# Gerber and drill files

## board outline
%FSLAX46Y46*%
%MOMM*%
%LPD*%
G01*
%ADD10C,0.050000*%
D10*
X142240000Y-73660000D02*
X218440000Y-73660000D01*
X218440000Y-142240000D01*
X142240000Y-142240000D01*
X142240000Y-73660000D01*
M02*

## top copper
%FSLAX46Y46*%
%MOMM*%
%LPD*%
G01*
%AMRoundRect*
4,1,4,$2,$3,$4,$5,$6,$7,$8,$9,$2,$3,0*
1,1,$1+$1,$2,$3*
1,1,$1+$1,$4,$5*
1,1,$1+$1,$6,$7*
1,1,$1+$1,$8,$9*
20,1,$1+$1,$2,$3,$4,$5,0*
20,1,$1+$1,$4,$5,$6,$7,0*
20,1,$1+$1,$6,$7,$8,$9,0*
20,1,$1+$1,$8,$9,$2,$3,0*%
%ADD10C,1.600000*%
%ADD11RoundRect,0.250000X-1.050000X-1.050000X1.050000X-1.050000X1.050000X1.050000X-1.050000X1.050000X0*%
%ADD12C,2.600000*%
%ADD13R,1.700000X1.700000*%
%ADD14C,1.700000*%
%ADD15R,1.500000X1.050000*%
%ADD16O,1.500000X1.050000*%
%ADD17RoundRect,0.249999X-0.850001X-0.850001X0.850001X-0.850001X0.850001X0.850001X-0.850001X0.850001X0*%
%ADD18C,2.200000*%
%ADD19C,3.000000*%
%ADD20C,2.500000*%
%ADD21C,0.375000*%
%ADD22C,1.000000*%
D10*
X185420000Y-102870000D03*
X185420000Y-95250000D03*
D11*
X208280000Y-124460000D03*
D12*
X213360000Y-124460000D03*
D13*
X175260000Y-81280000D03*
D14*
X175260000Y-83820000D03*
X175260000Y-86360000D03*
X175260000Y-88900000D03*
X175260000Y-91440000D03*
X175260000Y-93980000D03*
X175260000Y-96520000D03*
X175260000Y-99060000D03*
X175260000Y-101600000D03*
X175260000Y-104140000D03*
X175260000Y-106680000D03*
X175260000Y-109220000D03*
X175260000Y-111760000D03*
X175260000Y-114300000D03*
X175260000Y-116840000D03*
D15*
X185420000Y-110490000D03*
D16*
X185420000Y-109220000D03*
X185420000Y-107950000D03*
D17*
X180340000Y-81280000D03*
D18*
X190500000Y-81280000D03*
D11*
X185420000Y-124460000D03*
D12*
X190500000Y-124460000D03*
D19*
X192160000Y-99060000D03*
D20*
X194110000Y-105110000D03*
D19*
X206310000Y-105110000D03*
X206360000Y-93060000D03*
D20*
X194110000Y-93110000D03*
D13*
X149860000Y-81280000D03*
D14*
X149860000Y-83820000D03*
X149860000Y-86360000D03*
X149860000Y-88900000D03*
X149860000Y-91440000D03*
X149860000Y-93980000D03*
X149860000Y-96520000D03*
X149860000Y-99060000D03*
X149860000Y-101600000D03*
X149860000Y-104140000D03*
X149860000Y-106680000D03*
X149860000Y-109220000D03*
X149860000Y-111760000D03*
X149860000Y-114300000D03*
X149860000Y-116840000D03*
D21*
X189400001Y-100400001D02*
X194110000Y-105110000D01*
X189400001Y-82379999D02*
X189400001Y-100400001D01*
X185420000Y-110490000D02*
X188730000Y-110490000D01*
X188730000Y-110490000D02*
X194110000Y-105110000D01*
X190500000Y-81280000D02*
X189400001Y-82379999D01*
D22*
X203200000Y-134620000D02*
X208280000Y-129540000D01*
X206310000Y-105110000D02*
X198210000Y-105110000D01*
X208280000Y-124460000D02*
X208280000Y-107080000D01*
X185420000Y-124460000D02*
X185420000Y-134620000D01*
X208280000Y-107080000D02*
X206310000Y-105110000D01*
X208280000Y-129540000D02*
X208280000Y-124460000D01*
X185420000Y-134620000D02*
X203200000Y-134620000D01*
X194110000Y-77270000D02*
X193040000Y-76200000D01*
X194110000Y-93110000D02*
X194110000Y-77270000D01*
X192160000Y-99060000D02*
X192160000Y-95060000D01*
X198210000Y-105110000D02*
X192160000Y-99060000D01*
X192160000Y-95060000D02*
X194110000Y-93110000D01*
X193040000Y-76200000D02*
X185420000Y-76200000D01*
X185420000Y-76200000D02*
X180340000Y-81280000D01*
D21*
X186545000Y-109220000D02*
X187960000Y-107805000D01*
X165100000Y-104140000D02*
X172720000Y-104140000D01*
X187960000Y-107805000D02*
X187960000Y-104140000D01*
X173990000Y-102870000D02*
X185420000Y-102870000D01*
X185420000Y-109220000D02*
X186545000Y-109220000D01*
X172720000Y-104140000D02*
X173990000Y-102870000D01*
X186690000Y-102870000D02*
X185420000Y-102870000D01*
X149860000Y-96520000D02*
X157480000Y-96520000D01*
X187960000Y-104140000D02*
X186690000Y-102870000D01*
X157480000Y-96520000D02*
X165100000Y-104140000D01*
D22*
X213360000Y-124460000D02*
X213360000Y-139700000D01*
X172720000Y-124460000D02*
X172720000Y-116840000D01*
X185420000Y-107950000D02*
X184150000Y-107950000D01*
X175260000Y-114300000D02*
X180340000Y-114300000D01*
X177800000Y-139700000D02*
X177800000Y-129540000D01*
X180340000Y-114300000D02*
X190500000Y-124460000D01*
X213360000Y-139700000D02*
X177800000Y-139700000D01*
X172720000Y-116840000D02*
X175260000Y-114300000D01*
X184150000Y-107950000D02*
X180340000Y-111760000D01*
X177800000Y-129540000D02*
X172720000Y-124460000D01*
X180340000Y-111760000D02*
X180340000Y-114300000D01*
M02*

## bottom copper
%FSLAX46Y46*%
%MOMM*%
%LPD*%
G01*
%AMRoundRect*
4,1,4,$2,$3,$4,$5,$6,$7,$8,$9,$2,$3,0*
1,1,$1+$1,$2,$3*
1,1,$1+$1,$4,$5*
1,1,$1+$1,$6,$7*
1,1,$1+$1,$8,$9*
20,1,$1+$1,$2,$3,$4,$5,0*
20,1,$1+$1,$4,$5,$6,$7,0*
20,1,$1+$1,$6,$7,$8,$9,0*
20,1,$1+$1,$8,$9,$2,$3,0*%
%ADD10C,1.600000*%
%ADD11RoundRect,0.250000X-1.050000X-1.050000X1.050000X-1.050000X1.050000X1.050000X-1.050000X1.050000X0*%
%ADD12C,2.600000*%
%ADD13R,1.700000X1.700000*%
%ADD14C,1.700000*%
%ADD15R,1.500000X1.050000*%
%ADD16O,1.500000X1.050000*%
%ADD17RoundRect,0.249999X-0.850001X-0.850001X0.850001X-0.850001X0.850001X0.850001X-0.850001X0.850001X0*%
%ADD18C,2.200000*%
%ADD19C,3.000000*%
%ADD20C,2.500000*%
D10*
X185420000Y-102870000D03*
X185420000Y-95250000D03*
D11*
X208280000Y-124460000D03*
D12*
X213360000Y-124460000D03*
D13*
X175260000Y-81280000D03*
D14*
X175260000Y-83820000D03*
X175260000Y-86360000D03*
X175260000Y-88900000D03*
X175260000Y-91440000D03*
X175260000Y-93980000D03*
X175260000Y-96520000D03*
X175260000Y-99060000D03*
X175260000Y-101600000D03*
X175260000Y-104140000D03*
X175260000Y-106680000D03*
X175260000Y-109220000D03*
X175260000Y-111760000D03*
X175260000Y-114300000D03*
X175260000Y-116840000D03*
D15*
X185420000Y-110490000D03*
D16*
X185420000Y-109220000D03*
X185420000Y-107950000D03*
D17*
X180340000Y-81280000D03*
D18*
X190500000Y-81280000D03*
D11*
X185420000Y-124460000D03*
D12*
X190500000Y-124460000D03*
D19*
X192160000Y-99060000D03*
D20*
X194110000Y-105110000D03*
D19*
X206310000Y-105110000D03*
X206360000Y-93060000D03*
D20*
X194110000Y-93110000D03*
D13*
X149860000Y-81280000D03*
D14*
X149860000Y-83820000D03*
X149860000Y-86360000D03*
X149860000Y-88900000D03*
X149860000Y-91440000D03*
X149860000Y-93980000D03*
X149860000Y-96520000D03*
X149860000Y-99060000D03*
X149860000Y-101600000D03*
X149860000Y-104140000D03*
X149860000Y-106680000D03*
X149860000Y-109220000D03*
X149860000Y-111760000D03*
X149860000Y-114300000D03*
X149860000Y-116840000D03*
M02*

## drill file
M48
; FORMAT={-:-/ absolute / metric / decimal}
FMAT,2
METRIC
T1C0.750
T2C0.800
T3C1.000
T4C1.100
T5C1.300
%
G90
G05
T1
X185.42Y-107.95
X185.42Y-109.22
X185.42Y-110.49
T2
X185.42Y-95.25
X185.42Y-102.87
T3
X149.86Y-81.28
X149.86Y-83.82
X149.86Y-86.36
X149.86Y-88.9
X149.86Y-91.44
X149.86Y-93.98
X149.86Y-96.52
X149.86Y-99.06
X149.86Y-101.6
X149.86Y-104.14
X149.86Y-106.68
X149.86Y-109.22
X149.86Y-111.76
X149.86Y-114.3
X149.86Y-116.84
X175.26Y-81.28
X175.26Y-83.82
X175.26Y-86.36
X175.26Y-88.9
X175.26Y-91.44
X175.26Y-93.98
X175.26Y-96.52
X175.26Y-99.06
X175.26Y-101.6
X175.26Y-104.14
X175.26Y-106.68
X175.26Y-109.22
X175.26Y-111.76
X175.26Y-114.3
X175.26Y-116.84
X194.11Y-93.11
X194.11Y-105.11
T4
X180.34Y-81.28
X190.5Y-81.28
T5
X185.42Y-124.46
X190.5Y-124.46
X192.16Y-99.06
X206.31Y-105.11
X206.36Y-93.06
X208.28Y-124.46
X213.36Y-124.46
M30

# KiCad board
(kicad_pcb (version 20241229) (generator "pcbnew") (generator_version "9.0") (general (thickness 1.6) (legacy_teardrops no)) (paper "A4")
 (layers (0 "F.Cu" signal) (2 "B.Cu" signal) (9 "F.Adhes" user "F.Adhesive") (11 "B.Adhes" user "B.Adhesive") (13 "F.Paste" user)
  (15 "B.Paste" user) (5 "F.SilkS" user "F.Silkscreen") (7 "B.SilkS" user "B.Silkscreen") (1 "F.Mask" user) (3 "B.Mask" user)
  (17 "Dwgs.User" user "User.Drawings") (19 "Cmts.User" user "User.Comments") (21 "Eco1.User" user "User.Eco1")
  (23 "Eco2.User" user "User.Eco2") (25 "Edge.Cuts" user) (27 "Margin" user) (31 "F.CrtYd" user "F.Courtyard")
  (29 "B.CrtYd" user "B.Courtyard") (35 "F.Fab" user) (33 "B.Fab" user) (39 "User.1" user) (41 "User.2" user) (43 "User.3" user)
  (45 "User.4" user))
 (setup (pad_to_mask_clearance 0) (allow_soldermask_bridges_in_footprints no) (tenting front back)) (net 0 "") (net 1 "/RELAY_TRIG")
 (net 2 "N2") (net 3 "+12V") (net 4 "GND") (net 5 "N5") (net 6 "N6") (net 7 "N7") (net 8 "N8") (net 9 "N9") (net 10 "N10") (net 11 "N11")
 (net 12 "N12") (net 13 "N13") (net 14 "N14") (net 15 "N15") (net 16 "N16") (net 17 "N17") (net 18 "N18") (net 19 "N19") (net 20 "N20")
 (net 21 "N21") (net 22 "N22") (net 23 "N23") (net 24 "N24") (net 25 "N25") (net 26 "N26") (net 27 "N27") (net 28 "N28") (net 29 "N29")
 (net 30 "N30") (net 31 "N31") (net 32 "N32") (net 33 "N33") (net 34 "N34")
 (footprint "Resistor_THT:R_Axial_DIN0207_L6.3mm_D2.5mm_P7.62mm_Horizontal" (layer "F.Cu") (at 185.42 102.87 90)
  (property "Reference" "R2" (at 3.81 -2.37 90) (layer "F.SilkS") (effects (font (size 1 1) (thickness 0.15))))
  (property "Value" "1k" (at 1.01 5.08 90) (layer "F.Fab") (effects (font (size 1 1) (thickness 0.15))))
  (pad "1" thru_hole circle (at 0 0 90) (size 1.6 1.6) (drill 0.8) (layers "*.Cu" "*.Mask") (remove_unused_layers no) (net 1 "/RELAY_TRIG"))
  (pad "2" thru_hole circle (at 7.62 0 90) (size 1.6 1.6) (drill 0.8) (layers "*.Cu" "*.Mask") (remove_unused_layers no) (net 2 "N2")))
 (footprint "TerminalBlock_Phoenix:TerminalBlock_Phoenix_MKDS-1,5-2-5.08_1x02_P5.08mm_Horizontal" (layer "F.Cu") (at 208.28 124.46)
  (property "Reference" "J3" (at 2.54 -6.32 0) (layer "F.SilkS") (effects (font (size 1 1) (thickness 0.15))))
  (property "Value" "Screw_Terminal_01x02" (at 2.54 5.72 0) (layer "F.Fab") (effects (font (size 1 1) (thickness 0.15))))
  (pad "1" thru_hole roundrect (at 0 0) (size 2.6 2.6) (drill 1.3) (layers "*.Cu" "*.Mask") (remove_unused_layers no)
   (roundrect_rratio 0.096154) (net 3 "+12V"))
  (pad "2" thru_hole circle (at 5.08 0) (size 2.6 2.6) (drill 1.3) (layers "*.Cu" "*.Mask") (remove_unused_layers no) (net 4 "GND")))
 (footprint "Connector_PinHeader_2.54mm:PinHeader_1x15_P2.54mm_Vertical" (layer "F.Cu") (at 175.26 81.28)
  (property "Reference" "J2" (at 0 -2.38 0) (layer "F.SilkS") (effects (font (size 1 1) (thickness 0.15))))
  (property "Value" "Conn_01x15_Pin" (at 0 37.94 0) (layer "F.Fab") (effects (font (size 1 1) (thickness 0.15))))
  (pad "1" thru_hole rect (at 0 0) (size 1.7 1.7) (drill 1) (layers "*.Cu" "*.Mask") (remove_unused_layers no) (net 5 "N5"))
  (pad "2" thru_hole circle (at 0 2.54) (size 1.7 1.7) (drill 1) (layers "*.Cu" "*.Mask") (remove_unused_layers no) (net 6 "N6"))
  (pad "3" thru_hole circle (at 0 5.08) (size 1.7 1.7) (drill 1) (layers "*.Cu" "*.Mask") (remove_unused_layers no) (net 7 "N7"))
  (pad "4" thru_hole circle (at 0 7.62) (size 1.7 1.7) (drill 1) (layers "*.Cu" "*.Mask") (remove_unused_layers no) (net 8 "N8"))
  (pad "5" thru_hole circle (at 0 10.16) (size 1.7 1.7) (drill 1) (layers "*.Cu" "*.Mask") (remove_unused_layers no) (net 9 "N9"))
  (pad "6" thru_hole circle (at 0 12.7) (size 1.7 1.7) (drill 1) (layers "*.Cu" "*.Mask") (remove_unused_layers no) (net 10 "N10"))
  (pad "7" thru_hole circle (at 0 15.24) (size 1.7 1.7) (drill 1) (layers "*.Cu" "*.Mask") (remove_unused_layers no) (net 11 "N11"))
  (pad "8" thru_hole circle (at 0 17.78) (size 1.7 1.7) (drill 1) (layers "*.Cu" "*.Mask") (remove_unused_layers no) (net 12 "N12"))
  (pad "9" thru_hole circle (at 0 20.32) (size 1.7 1.7) (drill 1) (layers "*.Cu" "*.Mask") (remove_unused_layers no) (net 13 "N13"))
  (pad "10" thru_hole circle (at 0 22.86) (size 1.7 1.7) (drill 1) (layers "*.Cu" "*.Mask") (remove_unused_layers no) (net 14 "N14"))
  (pad "11" thru_hole circle (at 0 25.4) (size 1.7 1.7) (drill 1) (layers "*.Cu" "*.Mask") (remove_unused_layers no) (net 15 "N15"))
  (pad "12" thru_hole circle (at 0 27.94) (size 1.7 1.7) (drill 1) (layers "*.Cu" "*.Mask") (remove_unused_layers no) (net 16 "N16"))
  (pad "13" thru_hole circle (at 0 30.48) (size 1.7 1.7) (drill 1) (layers "*.Cu" "*.Mask") (remove_unused_layers no) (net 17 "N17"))
  (pad "14" thru_hole circle (at 0 33.02) (size 1.7 1.7) (drill 1) (layers "*.Cu" "*.Mask") (remove_unused_layers no) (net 4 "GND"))
  (pad "15" thru_hole circle (at 0 35.56) (size 1.7 1.7) (drill 1) (layers "*.Cu" "*.Mask") (remove_unused_layers no) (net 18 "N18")))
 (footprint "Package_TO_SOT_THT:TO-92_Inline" (layer "F.Cu") (at 185.42 110.49 90)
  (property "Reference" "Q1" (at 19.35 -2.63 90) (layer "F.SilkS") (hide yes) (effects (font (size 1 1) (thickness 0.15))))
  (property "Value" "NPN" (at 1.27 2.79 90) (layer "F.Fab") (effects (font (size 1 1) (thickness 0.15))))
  (pad "1" thru_hole rect (at 0 0 90) (size 1.05 1.5) (drill 0.75) (layers "*.Cu" "*.Mask") (remove_unused_layers no) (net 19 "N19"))
  (pad "2" thru_hole oval (at 1.27 0 90) (size 1.05 1.5) (drill 0.75) (layers "*.Cu" "*.Mask") (remove_unused_layers no)
   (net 1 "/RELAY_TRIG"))
  (pad "3" thru_hole oval (at 2.54 0 90) (size 1.05 1.5) (drill 0.75) (layers "*.Cu" "*.Mask") (remove_unused_layers no) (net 4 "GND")))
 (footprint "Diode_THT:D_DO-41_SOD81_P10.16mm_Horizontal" (layer "F.Cu") (at 180.34 81.28)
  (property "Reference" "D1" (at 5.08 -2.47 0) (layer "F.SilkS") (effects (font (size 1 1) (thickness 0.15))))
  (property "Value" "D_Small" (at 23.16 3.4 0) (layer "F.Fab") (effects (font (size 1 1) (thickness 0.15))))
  (pad "1" thru_hole roundrect (at 0 0) (size 2.2 2.2) (drill 1.1) (layers "*.Cu" "*.Mask") (remove_unused_layers no)
   (roundrect_rratio 0.113636) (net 3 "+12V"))
  (pad "2" thru_hole circle (at 10.16 0) (size 2.2 2.2) (drill 1.1) (layers "*.Cu" "*.Mask") (remove_unused_layers no) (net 19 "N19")))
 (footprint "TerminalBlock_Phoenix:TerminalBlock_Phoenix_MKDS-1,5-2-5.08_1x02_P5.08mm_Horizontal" (layer "F.Cu") (at 185.42 124.46)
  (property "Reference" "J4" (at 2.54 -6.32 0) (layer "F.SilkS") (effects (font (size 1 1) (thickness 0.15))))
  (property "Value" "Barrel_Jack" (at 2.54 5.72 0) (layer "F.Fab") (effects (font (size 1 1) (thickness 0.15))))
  (pad "1" thru_hole roundrect (at 0 0) (size 2.6 2.6) (drill 1.3) (layers "*.Cu" "*.Mask") (remove_unused_layers no)
   (roundrect_rratio 0.096154) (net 3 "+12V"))
  (pad "2" thru_hole circle (at 5.08 0) (size 2.6 2.6) (drill 1.3) (layers "*.Cu" "*.Mask") (remove_unused_layers no) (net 4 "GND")))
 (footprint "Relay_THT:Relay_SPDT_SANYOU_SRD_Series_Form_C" (layer "F.Cu") (at 192.16 99.06)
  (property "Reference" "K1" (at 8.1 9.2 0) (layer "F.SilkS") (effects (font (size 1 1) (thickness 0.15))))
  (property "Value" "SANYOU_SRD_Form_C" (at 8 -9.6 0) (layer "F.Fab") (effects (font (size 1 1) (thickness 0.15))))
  (pad "1" thru_hole circle (at 0 0 90) (size 3 3) (drill 1.3) (layers "*.Cu" "*.Mask") (remove_unused_layers no) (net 3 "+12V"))
  (pad "2" thru_hole circle (at 1.95 6.05 90) (size 2.5 2.5) (drill 1) (layers "*.Cu" "*.Mask") (remove_unused_layers no) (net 19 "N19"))
  (pad "3" thru_hole circle (at 14.15 6.05 90) (size 3 3) (drill 1.3) (layers "*.Cu" "*.Mask") (remove_unused_layers no) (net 3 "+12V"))
  (pad "4" thru_hole circle (at 14.2 -6 90) (size 3 3) (drill 1.3) (layers "*.Cu" "*.Mask") (remove_unused_layers no) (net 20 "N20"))
  (pad "5" thru_hole circle (at 1.95 -5.95 90) (size 2.5 2.5) (drill 1) (layers "*.Cu" "*.Mask") (remove_unused_layers no) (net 3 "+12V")))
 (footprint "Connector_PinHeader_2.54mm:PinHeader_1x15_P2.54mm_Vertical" (layer "F.Cu") (at 149.86 81.28)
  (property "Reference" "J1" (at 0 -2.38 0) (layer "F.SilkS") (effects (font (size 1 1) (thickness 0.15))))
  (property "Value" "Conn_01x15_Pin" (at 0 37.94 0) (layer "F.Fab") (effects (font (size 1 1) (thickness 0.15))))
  (pad "1" thru_hole rect (at 0 0) (size 1.7 1.7) (drill 1) (layers "*.Cu" "*.Mask") (remove_unused_layers no) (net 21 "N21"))
  (pad "2" thru_hole circle (at 0 2.54) (size 1.7 1.7) (drill 1) (layers "*.Cu" "*.Mask") (remove_unused_layers no) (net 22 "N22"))
  (pad "3" thru_hole circle (at 0 5.08) (size 1.7 1.7) (drill 1) (layers "*.Cu" "*.Mask") (remove_unused_layers no) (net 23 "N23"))
  (pad "4" thru_hole circle (at 0 7.62) (size 1.7 1.7) (drill 1) (layers "*.Cu" "*.Mask") (remove_unused_layers no) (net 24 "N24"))
  (pad "5" thru_hole circle (at 0 10.16) (size 1.7 1.7) (drill 1) (layers "*.Cu" "*.Mask") (remove_unused_layers no) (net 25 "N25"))
  (pad "6" thru_hole circle (at 0 12.7) (size 1.7 1.7) (drill 1) (layers "*.Cu" "*.Mask") (remove_unused_layers no) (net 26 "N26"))
  (pad "7" thru_hole circle (at 0 15.24) (size 1.7 1.7) (drill 1) (layers "*.Cu" "*.Mask") (remove_unused_layers no) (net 1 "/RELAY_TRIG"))
  (pad "8" thru_hole circle (at 0 17.78) (size 1.7 1.7) (drill 1) (layers "*.Cu" "*.Mask") (remove_unused_layers no) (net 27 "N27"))
  (pad "9" thru_hole circle (at 0 20.32) (size 1.7 1.7) (drill 1) (layers "*.Cu" "*.Mask") (remove_unused_layers no) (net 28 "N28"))
  (pad "10" thru_hole circle (at 0 22.86) (size 1.7 1.7) (drill 1) (layers "*.Cu" "*.Mask") (remove_unused_layers no) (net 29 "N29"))
  (pad "11" thru_hole circle (at 0 25.4) (size 1.7 1.7) (drill 1) (layers "*.Cu" "*.Mask") (remove_unused_layers no) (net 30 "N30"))
  (pad "12" thru_hole circle (at 0 27.94) (size 1.7 1.7) (drill 1) (layers "*.Cu" "*.Mask") (remove_unused_layers no) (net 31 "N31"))
  (pad "13" thru_hole circle (at 0 30.48) (size 1.7 1.7) (drill 1) (layers "*.Cu" "*.Mask") (remove_unused_layers no) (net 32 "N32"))
  (pad "14" thru_hole circle (at 0 33.02) (size 1.7 1.7) (drill 1) (layers "*.Cu" "*.Mask") (remove_unused_layers no) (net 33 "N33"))
  (pad "15" thru_hole circle (at 0 35.56) (size 1.7 1.7) (drill 1) (layers "*.Cu" "*.Mask") (remove_unused_layers no) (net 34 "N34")))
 (gr_rect (start 142.24 73.66) (end 218.44 142.24) (stroke (width 0.05) (type default)) (fill no) (layer "Edge.Cuts"))
 (segment (start 189.400001 100.400001) (end 194.11 105.11) (width 0.375) (layer "F.Cu") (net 19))
 (segment (start 189.400001 82.379999) (end 189.400001 100.400001) (width 0.375) (layer "F.Cu") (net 19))
 (segment (start 185.42 110.49) (end 188.73 110.49) (width 0.375) (layer "F.Cu") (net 19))
 (segment (start 188.73 110.49) (end 194.11 105.11) (width 0.375) (layer "F.Cu") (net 19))
 (segment (start 190.5 81.28) (end 189.400001 82.379999) (width 0.375) (layer "F.Cu") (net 19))
 (segment (start 203.2 134.62) (end 208.28 129.54) (width 1) (layer "F.Cu") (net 3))
 (segment (start 206.31 105.11) (end 198.21 105.11) (width 1) (layer "F.Cu") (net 3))
 (segment (start 208.28 124.46) (end 208.28 107.08) (width 1) (layer "F.Cu") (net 3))
 (segment (start 185.42 124.46) (end 185.42 134.62) (width 1) (layer "F.Cu") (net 3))
 (segment (start 208.28 107.08) (end 206.31 105.11) (width 1) (layer "F.Cu") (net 3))
 (segment (start 208.28 129.54) (end 208.28 124.46) (width 1) (layer "F.Cu") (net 3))
 (segment (start 185.42 134.62) (end 203.2 134.62) (width 1) (layer "F.Cu") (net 3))
 (segment (start 194.11 77.27) (end 193.04 76.2) (width 1) (layer "F.Cu") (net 3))
 (segment (start 194.11 93.11) (end 194.11 77.27) (width 1) (layer "F.Cu") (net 3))
 (segment (start 192.16 99.06) (end 192.16 95.06) (width 1) (layer "F.Cu") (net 3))
 (segment (start 198.21 105.11) (end 192.16 99.06) (width 1) (layer "F.Cu") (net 3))
 (segment (start 192.16 95.06) (end 194.11 93.11) (width 1) (layer "F.Cu") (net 3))
 (segment (start 193.04 76.2) (end 185.42 76.2) (width 1) (layer "F.Cu") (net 3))
 (segment (start 185.42 76.2) (end 180.34 81.28) (width 1) (layer "F.Cu") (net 3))
 (segment (start 186.545 109.22) (end 187.96 107.805) (width 0.375) (layer "F.Cu") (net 1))
 (segment (start 165.1 104.14) (end 172.72 104.14) (width 0.375) (layer "F.Cu") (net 1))
 (segment (start 187.96 107.805) (end 187.96 104.14) (width 0.375) (layer "F.Cu") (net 1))
 (segment (start 173.99 102.87) (end 185.42 102.87) (width 0.375) (layer "F.Cu") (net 1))
 (segment (start 185.42 109.22) (end 186.545 109.22) (width 0.375) (layer "F.Cu") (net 1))
 (segment (start 172.72 104.14) (end 173.99 102.87) (width 0.375) (layer "F.Cu") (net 1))
 (segment (start 186.69 102.87) (end 185.42 102.87) (width 0.375) (layer "F.Cu") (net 1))
 (segment (start 149.86 96.52) (end 157.48 96.52) (width 0.375) (layer "F.Cu") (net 1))
 (segment (start 187.96 104.14) (end 186.69 102.87) (width 0.375) (layer "F.Cu") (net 1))
 (segment (start 157.48 96.52) (end 165.1 104.14) (width 0.375) (layer "F.Cu") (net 1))
 (segment (start 213.36 124.46) (end 213.36 139.7) (width 1) (layer "F.Cu") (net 4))
 (segment (start 172.72 124.46) (end 172.72 116.84) (width 1) (layer "F.Cu") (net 4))
 (segment (start 185.42 107.95) (end 184.15 107.95) (width 1) (layer "F.Cu") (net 4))
 (segment (start 175.26 114.3) (end 180.34 114.3) (width 1) (layer "F.Cu") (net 4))
 (segment (start 177.8 139.7) (end 177.8 129.54) (width 1) (layer "F.Cu") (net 4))
 (segment (start 180.34 114.3) (end 190.5 124.46) (width 1) (layer "F.Cu") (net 4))
 (segment (start 213.36 139.7) (end 177.8 139.7) (width 1) (layer "F.Cu") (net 4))
 (segment (start 172.72 116.84) (end 175.26 114.3) (width 1) (layer "F.Cu") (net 4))
 (segment (start 184.15 107.95) (end 180.34 111.76) (width 1) (layer "F.Cu") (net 4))
 (segment (start 177.8 129.54) (end 172.72 124.46) (width 1) (layer "F.Cu") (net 4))
 (segment (start 180.34 111.76) (end 180.34 114.3) (width 1) (layer "F.Cu") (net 4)))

